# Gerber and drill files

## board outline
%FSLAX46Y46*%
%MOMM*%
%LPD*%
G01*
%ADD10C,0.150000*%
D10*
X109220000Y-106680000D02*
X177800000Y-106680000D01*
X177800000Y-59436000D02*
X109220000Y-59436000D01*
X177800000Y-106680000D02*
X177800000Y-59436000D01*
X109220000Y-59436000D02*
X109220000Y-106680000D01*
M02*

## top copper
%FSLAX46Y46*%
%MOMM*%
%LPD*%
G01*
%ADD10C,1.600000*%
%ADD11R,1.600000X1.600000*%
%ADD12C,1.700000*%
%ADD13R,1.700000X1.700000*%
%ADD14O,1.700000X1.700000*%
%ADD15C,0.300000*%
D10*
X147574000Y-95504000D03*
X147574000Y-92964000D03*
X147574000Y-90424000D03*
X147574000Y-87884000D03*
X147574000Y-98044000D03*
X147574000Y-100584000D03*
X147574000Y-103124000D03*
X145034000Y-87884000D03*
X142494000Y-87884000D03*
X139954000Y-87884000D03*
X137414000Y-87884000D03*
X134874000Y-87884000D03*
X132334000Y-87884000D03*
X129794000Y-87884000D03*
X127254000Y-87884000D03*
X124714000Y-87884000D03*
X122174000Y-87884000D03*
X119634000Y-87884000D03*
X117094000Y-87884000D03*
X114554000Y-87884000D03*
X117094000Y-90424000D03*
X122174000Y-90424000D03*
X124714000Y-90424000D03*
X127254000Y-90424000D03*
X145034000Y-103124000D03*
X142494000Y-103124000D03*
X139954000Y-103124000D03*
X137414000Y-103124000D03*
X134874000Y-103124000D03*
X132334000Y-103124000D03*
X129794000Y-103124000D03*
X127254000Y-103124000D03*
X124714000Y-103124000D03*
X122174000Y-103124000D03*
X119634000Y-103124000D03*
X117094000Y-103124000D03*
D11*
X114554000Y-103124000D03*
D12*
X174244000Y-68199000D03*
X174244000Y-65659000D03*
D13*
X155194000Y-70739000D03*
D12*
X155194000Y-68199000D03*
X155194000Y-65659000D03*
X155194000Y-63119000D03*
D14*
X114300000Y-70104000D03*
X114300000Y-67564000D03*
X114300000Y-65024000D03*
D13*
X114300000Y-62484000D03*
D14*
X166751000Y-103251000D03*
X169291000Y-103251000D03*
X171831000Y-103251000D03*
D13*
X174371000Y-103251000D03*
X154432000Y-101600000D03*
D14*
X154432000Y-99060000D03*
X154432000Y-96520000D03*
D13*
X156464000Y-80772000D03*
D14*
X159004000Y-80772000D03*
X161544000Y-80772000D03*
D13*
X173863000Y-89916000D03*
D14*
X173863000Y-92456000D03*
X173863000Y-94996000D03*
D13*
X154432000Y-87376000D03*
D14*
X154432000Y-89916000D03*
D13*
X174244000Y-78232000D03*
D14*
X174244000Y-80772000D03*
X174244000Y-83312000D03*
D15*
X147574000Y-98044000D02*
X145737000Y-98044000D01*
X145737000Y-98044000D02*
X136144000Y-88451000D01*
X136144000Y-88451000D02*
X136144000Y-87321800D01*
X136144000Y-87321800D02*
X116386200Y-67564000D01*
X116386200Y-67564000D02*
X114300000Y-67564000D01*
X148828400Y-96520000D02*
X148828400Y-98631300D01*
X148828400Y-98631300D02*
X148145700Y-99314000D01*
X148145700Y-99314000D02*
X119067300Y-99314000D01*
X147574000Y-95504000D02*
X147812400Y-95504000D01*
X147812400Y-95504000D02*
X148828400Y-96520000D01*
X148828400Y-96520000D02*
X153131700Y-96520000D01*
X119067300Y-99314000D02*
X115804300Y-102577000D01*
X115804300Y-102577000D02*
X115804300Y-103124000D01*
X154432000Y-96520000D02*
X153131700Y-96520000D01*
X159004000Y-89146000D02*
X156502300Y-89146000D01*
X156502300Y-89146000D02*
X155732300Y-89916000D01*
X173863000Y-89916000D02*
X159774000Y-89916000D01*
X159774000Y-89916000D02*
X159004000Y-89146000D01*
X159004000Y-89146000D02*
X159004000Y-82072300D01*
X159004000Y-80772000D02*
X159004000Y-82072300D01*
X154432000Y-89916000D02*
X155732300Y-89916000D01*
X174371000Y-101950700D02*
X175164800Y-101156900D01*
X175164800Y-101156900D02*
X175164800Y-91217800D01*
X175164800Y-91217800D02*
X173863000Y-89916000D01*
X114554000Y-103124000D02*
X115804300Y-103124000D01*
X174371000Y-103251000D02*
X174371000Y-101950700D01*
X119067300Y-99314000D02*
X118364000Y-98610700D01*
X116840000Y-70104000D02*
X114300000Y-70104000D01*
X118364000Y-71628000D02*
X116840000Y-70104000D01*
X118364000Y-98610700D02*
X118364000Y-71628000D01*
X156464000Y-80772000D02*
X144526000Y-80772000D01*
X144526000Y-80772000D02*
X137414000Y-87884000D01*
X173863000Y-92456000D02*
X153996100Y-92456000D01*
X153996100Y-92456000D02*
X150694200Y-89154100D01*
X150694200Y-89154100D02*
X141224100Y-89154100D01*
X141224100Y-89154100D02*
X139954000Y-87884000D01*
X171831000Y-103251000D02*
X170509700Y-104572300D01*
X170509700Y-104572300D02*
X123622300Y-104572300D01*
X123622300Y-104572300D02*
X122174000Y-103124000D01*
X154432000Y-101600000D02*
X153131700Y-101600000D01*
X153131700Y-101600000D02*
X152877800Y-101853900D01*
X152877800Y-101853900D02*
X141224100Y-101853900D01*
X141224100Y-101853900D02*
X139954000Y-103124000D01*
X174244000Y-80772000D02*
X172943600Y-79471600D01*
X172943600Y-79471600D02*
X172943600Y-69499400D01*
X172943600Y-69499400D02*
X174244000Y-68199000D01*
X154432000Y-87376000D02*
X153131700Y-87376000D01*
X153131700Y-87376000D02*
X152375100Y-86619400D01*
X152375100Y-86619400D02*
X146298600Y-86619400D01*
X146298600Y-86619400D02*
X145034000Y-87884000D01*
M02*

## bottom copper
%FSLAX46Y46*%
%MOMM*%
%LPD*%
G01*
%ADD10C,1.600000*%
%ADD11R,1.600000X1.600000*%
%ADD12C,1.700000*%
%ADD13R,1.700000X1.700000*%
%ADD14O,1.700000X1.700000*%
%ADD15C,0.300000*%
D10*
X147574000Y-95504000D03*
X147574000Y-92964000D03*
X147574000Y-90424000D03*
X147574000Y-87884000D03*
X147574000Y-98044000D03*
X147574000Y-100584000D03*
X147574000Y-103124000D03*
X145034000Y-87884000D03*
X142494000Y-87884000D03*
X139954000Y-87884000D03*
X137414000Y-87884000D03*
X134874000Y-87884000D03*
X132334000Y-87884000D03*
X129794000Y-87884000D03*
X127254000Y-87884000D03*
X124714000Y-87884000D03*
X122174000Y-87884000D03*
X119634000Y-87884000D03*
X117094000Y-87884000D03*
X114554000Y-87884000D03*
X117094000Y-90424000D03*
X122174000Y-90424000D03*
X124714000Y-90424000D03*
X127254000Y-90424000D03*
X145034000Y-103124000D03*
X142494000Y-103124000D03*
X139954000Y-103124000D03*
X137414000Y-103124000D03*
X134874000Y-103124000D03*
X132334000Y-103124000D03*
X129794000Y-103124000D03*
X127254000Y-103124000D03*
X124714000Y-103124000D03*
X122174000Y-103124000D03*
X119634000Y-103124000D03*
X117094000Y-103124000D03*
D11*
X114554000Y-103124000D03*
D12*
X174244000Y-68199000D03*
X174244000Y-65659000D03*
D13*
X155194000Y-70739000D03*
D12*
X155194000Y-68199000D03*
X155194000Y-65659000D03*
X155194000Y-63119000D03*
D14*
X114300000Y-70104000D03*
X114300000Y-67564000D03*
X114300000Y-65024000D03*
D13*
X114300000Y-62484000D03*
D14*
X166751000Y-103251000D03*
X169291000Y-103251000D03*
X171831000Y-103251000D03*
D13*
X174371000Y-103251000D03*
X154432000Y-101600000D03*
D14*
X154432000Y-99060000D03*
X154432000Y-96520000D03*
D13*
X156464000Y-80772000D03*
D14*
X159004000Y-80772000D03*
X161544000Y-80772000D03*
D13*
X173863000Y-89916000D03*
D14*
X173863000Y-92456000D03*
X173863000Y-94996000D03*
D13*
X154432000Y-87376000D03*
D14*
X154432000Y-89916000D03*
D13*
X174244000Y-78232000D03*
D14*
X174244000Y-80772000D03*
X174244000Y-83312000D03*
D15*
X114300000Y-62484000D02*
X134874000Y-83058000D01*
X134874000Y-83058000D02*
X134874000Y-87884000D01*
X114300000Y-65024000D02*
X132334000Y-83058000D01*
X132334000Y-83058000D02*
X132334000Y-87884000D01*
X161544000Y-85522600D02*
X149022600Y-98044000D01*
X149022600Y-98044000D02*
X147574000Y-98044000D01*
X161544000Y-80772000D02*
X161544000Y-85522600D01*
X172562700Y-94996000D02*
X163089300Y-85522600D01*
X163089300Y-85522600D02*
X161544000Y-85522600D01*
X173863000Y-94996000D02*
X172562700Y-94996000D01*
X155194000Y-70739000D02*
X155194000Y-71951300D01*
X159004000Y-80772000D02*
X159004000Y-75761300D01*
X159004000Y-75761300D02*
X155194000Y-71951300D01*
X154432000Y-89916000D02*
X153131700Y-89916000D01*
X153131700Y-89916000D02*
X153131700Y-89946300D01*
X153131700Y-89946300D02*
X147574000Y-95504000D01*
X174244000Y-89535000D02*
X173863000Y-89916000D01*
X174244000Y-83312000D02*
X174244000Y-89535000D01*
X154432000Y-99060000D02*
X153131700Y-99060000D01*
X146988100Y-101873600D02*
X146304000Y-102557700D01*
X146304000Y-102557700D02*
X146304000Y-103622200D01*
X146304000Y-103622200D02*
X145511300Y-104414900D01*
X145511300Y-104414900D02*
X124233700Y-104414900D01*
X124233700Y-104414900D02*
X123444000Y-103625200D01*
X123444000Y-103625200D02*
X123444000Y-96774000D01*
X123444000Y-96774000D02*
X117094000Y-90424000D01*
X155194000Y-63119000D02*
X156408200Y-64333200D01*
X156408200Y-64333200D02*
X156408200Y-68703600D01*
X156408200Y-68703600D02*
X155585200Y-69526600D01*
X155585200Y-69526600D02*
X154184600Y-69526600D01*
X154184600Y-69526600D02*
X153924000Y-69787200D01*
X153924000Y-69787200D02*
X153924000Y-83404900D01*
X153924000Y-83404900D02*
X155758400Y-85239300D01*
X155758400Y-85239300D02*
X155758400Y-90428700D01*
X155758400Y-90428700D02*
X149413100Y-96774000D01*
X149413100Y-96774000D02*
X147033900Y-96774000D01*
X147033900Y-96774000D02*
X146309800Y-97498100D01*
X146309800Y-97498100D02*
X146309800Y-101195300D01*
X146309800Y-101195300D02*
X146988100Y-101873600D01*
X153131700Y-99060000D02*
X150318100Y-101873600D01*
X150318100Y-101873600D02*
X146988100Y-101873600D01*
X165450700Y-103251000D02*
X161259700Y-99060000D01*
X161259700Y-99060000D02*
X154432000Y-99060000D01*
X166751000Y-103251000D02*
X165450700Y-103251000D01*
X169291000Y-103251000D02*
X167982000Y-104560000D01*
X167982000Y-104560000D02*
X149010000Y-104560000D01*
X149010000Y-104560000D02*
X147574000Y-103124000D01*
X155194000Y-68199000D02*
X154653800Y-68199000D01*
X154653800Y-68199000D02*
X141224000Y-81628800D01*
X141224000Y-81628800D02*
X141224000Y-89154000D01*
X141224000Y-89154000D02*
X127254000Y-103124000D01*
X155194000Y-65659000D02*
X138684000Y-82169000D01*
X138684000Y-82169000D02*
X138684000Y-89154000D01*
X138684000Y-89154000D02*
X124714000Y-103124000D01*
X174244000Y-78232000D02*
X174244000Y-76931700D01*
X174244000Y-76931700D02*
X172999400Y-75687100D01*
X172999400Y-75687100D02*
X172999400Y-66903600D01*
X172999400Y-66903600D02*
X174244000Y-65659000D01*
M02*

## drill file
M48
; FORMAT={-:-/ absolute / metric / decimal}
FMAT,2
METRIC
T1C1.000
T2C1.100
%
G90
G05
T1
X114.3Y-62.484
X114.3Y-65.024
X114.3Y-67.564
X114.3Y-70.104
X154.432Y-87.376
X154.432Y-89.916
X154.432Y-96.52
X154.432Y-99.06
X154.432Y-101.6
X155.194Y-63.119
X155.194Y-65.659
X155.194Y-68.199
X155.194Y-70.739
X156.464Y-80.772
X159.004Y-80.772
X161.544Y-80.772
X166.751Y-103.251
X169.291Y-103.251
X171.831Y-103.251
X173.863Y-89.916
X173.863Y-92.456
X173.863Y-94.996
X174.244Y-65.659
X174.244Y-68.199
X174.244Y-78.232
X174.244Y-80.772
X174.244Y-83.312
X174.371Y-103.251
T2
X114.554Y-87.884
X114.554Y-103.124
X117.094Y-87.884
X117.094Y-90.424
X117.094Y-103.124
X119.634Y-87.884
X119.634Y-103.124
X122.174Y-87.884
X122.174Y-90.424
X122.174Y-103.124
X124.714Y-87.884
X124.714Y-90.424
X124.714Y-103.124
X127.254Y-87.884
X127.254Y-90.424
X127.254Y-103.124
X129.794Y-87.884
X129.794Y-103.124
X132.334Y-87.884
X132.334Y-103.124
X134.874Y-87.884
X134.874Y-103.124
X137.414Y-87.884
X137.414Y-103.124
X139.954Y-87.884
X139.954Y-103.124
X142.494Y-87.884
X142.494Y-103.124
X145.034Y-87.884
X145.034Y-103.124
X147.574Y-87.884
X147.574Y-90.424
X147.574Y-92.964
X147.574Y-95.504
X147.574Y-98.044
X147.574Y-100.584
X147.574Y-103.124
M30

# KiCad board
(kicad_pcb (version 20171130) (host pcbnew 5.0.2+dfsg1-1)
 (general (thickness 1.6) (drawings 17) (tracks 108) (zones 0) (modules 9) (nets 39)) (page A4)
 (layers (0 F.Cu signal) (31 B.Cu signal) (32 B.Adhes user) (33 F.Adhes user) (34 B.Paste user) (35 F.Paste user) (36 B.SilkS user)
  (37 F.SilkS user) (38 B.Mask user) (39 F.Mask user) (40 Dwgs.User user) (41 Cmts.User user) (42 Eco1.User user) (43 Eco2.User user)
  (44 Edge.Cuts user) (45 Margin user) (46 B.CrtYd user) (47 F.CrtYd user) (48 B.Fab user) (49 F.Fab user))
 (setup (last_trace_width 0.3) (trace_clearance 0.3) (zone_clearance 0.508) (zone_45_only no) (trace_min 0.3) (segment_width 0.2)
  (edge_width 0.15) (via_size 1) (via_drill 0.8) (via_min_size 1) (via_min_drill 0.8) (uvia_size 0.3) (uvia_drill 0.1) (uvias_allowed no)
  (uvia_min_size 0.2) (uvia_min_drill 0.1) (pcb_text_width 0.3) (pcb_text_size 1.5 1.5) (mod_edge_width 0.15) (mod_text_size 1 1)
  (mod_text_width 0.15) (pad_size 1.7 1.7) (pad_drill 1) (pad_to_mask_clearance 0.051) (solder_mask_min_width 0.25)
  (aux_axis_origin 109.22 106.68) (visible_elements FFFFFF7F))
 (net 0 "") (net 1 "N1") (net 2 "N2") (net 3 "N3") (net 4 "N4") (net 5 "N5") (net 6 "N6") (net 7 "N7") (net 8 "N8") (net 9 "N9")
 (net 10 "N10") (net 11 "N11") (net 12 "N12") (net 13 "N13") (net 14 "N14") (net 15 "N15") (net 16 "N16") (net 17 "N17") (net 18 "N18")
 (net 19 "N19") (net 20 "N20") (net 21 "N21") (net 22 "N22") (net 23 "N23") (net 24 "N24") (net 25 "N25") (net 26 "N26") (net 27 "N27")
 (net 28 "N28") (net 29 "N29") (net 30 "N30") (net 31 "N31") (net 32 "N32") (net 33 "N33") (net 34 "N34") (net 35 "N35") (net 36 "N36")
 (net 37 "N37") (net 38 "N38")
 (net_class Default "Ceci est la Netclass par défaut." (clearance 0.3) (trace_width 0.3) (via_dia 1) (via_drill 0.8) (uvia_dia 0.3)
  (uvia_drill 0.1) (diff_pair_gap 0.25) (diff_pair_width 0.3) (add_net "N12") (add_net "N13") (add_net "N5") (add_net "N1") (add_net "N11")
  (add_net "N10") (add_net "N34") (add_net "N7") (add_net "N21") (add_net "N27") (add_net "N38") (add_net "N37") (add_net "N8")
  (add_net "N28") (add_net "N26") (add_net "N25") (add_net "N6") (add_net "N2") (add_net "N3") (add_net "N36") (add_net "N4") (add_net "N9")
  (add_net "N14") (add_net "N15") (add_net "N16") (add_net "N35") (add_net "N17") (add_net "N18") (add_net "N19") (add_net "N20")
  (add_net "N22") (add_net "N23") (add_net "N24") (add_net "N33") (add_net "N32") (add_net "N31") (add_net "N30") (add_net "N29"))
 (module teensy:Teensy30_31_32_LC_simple (layer F.Cu) (at 131.064 95.504)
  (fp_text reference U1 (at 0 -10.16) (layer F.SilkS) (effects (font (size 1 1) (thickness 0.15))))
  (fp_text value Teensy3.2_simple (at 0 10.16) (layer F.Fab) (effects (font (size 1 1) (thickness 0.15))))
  (pad 17 thru_hole circle (at 16.51 0) (size 1.6 1.6) (drill 1.1) (layers *.Cu *.Mask F.SilkS) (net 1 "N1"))
  (pad 18 thru_hole circle (at 16.51 -2.54) (size 1.6 1.6) (drill 1.1) (layers *.Cu *.Mask F.SilkS) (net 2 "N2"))
  (pad 19 thru_hole circle (at 16.51 -5.08) (size 1.6 1.6) (drill 1.1) (layers *.Cu *.Mask F.SilkS) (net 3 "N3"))
  (pad 20 thru_hole circle (at 16.51 -7.62) (size 1.6 1.6) (drill 1.1) (layers *.Cu *.Mask F.SilkS) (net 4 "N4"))
  (pad 16 thru_hole circle (at 16.51 2.54) (size 1.6 1.6) (drill 1.1) (layers *.Cu *.Mask F.SilkS) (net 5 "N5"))
  (pad 15 thru_hole circle (at 16.51 5.08) (size 1.6 1.6) (drill 1.1) (layers *.Cu *.Mask F.SilkS) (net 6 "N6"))
  (pad 14 thru_hole circle (at 16.51 7.62) (size 1.6 1.6) (drill 1.1) (layers *.Cu *.Mask F.SilkS) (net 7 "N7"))
  (pad 21 thru_hole circle (at 13.97 -7.62) (size 1.6 1.6) (drill 1.1) (layers *.Cu *.Mask F.SilkS) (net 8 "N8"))
  (pad 22 thru_hole circle (at 11.43 -7.62) (size 1.6 1.6) (drill 1.1) (layers *.Cu *.Mask F.SilkS) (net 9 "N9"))
  (pad 23 thru_hole circle (at 8.89 -7.62) (size 1.6 1.6) (drill 1.1) (layers *.Cu *.Mask F.SilkS) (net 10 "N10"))
  (pad 24 thru_hole circle (at 6.35 -7.62) (size 1.6 1.6) (drill 1.1) (layers *.Cu *.Mask F.SilkS) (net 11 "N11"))
  (pad 25 thru_hole circle (at 3.81 -7.62) (size 1.6 1.6) (drill 1.1) (layers *.Cu *.Mask F.SilkS) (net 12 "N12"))
  (pad 26 thru_hole circle (at 1.27 -7.62) (size 1.6 1.6) (drill 1.1) (layers *.Cu *.Mask F.SilkS) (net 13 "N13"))
  (pad 27 thru_hole circle (at -1.27 -7.62) (size 1.6 1.6) (drill 1.1) (layers *.Cu *.Mask F.SilkS) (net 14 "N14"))
  (pad 28 thru_hole circle (at -3.81 -7.62) (size 1.6 1.6) (drill 1.1) (layers *.Cu *.Mask F.SilkS) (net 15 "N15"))
  (pad 29 thru_hole circle (at -6.35 -7.62) (size 1.6 1.6) (drill 1.1) (layers *.Cu *.Mask F.SilkS) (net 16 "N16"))
  (pad 30 thru_hole circle (at -8.89 -7.62) (size 1.6 1.6) (drill 1.1) (layers *.Cu *.Mask F.SilkS) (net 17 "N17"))
  (pad 31 thru_hole circle (at -11.43 -7.62) (size 1.6 1.6) (drill 1.1) (layers *.Cu *.Mask F.SilkS) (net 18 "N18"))
  (pad 32 thru_hole circle (at -13.97 -7.62) (size 1.6 1.6) (drill 1.1) (layers *.Cu *.Mask F.SilkS) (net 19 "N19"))
  (pad 33 thru_hole circle (at -16.51 -7.62) (size 1.6 1.6) (drill 1.1) (layers *.Cu *.Mask F.SilkS) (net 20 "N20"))
  (pad 34 thru_hole circle (at -13.97 -5.08) (size 1.6 1.6) (drill 1.1) (layers *.Cu *.Mask F.SilkS) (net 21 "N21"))
  (pad 35 thru_hole circle (at -8.89 -5.08) (size 1.6 1.6) (drill 1.1) (layers *.Cu *.Mask F.SilkS) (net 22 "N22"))
  (pad 36 thru_hole circle (at -6.35 -5.08) (size 1.6 1.6) (drill 1.1) (layers *.Cu *.Mask F.SilkS) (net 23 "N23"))
  (pad 37 thru_hole circle (at -3.81 -5.08) (size 1.6 1.6) (drill 1.1) (layers *.Cu *.Mask F.SilkS) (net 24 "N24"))
  (pad 13 thru_hole circle (at 13.97 7.62) (size 1.6 1.6) (drill 1.1) (layers *.Cu *.Mask F.SilkS) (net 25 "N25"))
  (pad 12 thru_hole circle (at 11.43 7.62) (size 1.6 1.6) (drill 1.1) (layers *.Cu *.Mask F.SilkS) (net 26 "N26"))
  (pad 11 thru_hole circle (at 8.89 7.62) (size 1.6 1.6) (drill 1.1) (layers *.Cu *.Mask F.SilkS) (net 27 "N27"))
  (pad 10 thru_hole circle (at 6.35 7.62) (size 1.6 1.6) (drill 1.1) (layers *.Cu *.Mask F.SilkS) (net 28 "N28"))
  (pad 9 thru_hole circle (at 3.81 7.62) (size 1.6 1.6) (drill 1.1) (layers *.Cu *.Mask F.SilkS) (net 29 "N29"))
  (pad 8 thru_hole circle (at 1.27 7.62) (size 1.6 1.6) (drill 1.1) (layers *.Cu *.Mask F.SilkS) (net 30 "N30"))
  (pad 7 thru_hole circle (at -1.27 7.62) (size 1.6 1.6) (drill 1.1) (layers *.Cu *.Mask F.SilkS) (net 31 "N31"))
  (pad 6 thru_hole circle (at -3.81 7.62) (size 1.6 1.6) (drill 1.1) (layers *.Cu *.Mask F.SilkS) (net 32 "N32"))
  (pad 5 thru_hole circle (at -6.35 7.62) (size 1.6 1.6) (drill 1.1) (layers *.Cu *.Mask F.SilkS) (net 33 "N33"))
  (pad 4 thru_hole circle (at -8.89 7.62) (size 1.6 1.6) (drill 1.1) (layers *.Cu *.Mask F.SilkS) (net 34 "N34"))
  (pad 3 thru_hole circle (at -11.43 7.62) (size 1.6 1.6) (drill 1.1) (layers *.Cu *.Mask F.SilkS) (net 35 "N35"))
  (pad 2 thru_hole circle (at -13.97 7.62) (size 1.6 1.6) (drill 1.1) (layers *.Cu *.Mask F.SilkS) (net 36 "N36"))
  (pad 1 thru_hole rect (at -16.51 7.62) (size 1.6 1.6) (drill 1.1) (layers *.Cu *.Mask F.SilkS) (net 1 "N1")))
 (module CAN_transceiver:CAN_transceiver (layer F.Cu) (at 153.924 72.644)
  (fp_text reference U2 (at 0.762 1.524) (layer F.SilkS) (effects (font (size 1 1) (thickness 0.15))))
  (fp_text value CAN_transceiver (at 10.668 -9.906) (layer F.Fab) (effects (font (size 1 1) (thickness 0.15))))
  (pad 5 thru_hole circle (at 20.32 -4.445) (size 1.7 1.7) (drill 1) (layers *.Cu *.Mask) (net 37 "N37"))
  (pad 6 thru_hole circle (at 20.32 -6.985) (size 1.7 1.7) (drill 1) (layers *.Cu *.Mask) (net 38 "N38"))
  (pad 1 thru_hole rect (at 1.27 -1.905) (size 1.7 1.7) (drill 1) (layers *.Cu *.Mask) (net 1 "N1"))
  (pad 2 thru_hole circle (at 1.27 -4.445) (size 1.7 1.7) (drill 1) (layers *.Cu *.Mask) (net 32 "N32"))
  (pad 3 thru_hole circle (at 1.27 -6.985) (size 1.7 1.7) (drill 1) (layers *.Cu *.Mask) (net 33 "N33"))
  (pad 4 thru_hole circle (at 1.27 -9.525) (size 1.7 1.7) (drill 1) (layers *.Cu *.Mask) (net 21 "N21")))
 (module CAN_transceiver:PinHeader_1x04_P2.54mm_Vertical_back (layer F.Cu) (at 114.3 62.484)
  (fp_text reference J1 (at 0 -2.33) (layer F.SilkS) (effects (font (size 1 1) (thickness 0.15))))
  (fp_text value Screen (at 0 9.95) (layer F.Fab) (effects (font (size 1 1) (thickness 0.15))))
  (pad 4 thru_hole oval (at 0 7.62) (size 1.7 1.7) (drill 1) (layers *.Cu *.Mask) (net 1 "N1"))
  (pad 3 thru_hole oval (at 0 5.08) (size 1.7 1.7) (drill 1) (layers *.Cu *.Mask) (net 5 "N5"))
  (pad 2 thru_hole oval (at 0 2.54) (size 1.7 1.7) (drill 1) (layers *.Cu *.Mask) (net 13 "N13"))
  (pad 1 thru_hole rect (at 0 0) (size 1.7 1.7) (drill 1) (layers *.Cu *.Mask) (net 12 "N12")))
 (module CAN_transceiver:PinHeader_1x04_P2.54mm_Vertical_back (layer F.Cu) (at 174.371 103.251 270)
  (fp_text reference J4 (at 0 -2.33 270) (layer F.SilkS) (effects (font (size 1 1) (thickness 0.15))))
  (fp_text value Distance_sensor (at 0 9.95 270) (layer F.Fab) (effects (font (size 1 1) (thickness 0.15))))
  (pad 4 thru_hole oval (at 0 7.62 270) (size 1.7 1.7) (drill 1) (layers *.Cu *.Mask) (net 21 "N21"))
  (pad 3 thru_hole oval (at 0 5.08 270) (size 1.7 1.7) (drill 1) (layers *.Cu *.Mask) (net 7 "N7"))
  (pad 2 thru_hole oval (at 0 2.54 270) (size 1.7 1.7) (drill 1) (layers *.Cu *.Mask) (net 34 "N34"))
  (pad 1 thru_hole rect (at 0 0 270) (size 1.7 1.7) (drill 1) (layers *.Cu *.Mask) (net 1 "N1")))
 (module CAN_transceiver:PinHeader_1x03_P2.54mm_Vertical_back (layer F.Cu) (at 154.432 101.6 180)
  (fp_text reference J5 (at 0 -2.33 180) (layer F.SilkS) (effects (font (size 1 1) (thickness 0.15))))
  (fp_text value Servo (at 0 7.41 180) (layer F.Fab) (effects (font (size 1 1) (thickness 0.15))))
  (pad 1 thru_hole rect (at 0 0 180) (size 1.7 1.7) (drill 1) (layers *.Cu *.Mask) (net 27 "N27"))
  (pad 2 thru_hole oval (at 0 2.54 180) (size 1.7 1.7) (drill 1) (layers *.Cu *.Mask) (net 21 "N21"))
  (pad 3 thru_hole oval (at 0 5.08 180) (size 1.7 1.7) (drill 1) (layers *.Cu *.Mask) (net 1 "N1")))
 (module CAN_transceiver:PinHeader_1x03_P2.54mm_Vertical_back (layer F.Cu) (at 156.464 80.772 90)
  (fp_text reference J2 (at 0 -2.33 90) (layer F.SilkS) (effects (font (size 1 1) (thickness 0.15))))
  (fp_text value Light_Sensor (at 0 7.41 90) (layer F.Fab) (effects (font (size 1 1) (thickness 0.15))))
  (pad 1 thru_hole rect (at 0 0 90) (size 1.7 1.7) (drill 1) (layers *.Cu *.Mask) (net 11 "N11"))
  (pad 2 thru_hole oval (at 0 2.54 90) (size 1.7 1.7) (drill 1) (layers *.Cu *.Mask) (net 1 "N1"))
  (pad 3 thru_hole oval (at 0 5.08 90) (size 1.7 1.7) (drill 1) (layers *.Cu *.Mask) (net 5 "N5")))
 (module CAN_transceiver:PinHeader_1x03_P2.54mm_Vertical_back (layer F.Cu) (at 173.863 89.916)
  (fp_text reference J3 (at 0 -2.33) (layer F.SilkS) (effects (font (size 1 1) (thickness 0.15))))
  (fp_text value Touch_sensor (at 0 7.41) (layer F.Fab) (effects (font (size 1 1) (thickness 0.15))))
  (pad 1 thru_hole rect (at 0 0) (size 1.7 1.7) (drill 1) (layers *.Cu *.Mask) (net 1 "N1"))
  (pad 2 thru_hole oval (at 0 2.54) (size 1.7 1.7) (drill 1) (layers *.Cu *.Mask) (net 10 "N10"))
  (pad 3 thru_hole oval (at 0 5.08) (size 1.7 1.7) (drill 1) (layers *.Cu *.Mask) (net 5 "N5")))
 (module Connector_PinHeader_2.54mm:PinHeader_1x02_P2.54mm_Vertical (layer F.Cu) (at 154.432 87.376)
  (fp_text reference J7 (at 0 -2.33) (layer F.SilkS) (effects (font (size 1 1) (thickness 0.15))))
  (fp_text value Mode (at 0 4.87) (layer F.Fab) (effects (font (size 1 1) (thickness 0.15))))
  (pad 1 thru_hole rect (at 0 0) (size 1.7 1.7) (drill 1) (layers *.Cu *.Mask) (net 8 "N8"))
  (pad 2 thru_hole oval (at 0 2.54) (size 1.7 1.7) (drill 1) (layers *.Cu *.Mask) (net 1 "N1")))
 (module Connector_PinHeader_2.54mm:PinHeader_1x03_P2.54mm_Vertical (layer F.Cu) (at 174.244 78.232)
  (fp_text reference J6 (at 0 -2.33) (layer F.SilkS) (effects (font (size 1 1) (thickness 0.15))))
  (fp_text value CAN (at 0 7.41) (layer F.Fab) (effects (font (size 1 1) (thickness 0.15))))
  (pad 1 thru_hole rect (at 0 0) (size 1.7 1.7) (drill 1) (layers *.Cu *.Mask) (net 38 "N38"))
  (pad 2 thru_hole oval (at 0 2.54) (size 1.7 1.7) (drill 1) (layers *.Cu *.Mask) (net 37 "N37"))
  (pad 3 thru_hole oval (at 0 5.08) (size 1.7 1.7) (drill 1) (layers *.Cu *.Mask) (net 1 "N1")))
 (gr_line (start 109.22 106.68) (end 177.8 106.68) (layer Edge.Cuts) (width 0.15))
 (gr_line (start 177.8 59.436) (end 109.22 59.436) (layer Edge.Cuts) (width 0.15))
 (gr_line (start 177.8 106.68) (end 177.8 59.436) (layer Edge.Cuts) (width 0.15))
 (gr_line (start 109.22 59.436) (end 109.22 106.68) (layer Edge.Cuts) (width 0.15))
 (segment (start 114.3 62.484) (end 134.874 83.058) (width 0.3) (layer B.Cu) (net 12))
 (segment (start 134.874 83.058) (end 134.874 87.884) (width 0.3) (layer B.Cu) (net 12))
 (segment (start 114.3 65.024) (end 132.334 83.058) (width 0.3) (layer B.Cu) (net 13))
 (segment (start 132.334 83.058) (end 132.334 87.884) (width 0.3) (layer B.Cu) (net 13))
 (segment (start 161.544 85.5226) (end 149.0226 98.044) (width 0.3) (layer B.Cu) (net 5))
 (segment (start 149.0226 98.044) (end 147.574 98.044) (width 0.3) (layer B.Cu) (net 5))
 (segment (start 161.544 80.772) (end 161.544 85.5226) (width 0.3) (layer B.Cu) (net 5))
 (segment (start 172.5627 94.996) (end 163.0893 85.5226) (width 0.3) (layer B.Cu) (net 5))
 (segment (start 163.0893 85.5226) (end 161.544 85.5226) (width 0.3) (layer B.Cu) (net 5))
 (segment (start 173.863 94.996) (end 172.5627 94.996) (width 0.3) (layer B.Cu) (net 5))
 (segment (start 147.574 98.044) (end 145.737 98.044) (width 0.3) (layer F.Cu) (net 5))
 (segment (start 145.737 98.044) (end 136.144 88.451) (width 0.3) (layer F.Cu) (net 5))
 (segment (start 136.144 88.451) (end 136.144 87.3218) (width 0.3) (layer F.Cu) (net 5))
 (segment (start 136.144 87.3218) (end 116.3862 67.564) (width 0.3) (layer F.Cu) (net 5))
 (segment (start 116.3862 67.564) (end 114.3 67.564) (width 0.3) (layer F.Cu) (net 5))
 (segment (start 155.194 70.739) (end 155.194 71.9513) (width 0.3) (layer B.Cu) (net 1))
 (segment (start 159.004 80.772) (end 159.004 75.7613) (width 0.3) (layer B.Cu) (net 1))
 (segment (start 159.004 75.7613) (end 155.194 71.9513) (width 0.3) (layer B.Cu) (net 1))
 (segment (start 154.432 89.916) (end 153.1317 89.916) (width 0.3) (layer B.Cu) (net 1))
 (segment (start 153.1317 89.916) (end 153.1317 89.9463) (width 0.3) (layer B.Cu) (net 1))
 (segment (start 153.1317 89.9463) (end 147.574 95.504) (width 0.3) (layer B.Cu) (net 1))
 (segment (start 148.8284 96.52) (end 148.8284 98.6313) (width 0.3) (layer F.Cu) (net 1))
 (segment (start 148.8284 98.6313) (end 148.1457 99.314) (width 0.3) (layer F.Cu) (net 1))
 (segment (start 148.1457 99.314) (end 119.0673 99.314) (width 0.3) (layer F.Cu) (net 1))
 (segment (start 147.574 95.504) (end 147.8124 95.504) (width 0.3) (layer F.Cu) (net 1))
 (segment (start 147.8124 95.504) (end 148.8284 96.52) (width 0.3) (layer F.Cu) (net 1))
 (segment (start 148.8284 96.52) (end 153.1317 96.52) (width 0.3) (layer F.Cu) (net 1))
 (segment (start 119.0673 99.314) (end 115.8043 102.577) (width 0.3) (layer F.Cu) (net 1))
 (segment (start 115.8043 102.577) (end 115.8043 103.124) (width 0.3) (layer F.Cu) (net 1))
 (segment (start 154.432 96.52) (end 153.1317 96.52) (width 0.3) (layer F.Cu) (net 1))
 (segment (start 159.004 89.146) (end 156.5023 89.146) (width 0.3) (layer F.Cu) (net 1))
 (segment (start 156.5023 89.146) (end 155.7323 89.916) (width 0.3) (layer F.Cu) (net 1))
 (segment (start 173.863 89.916) (end 159.774 89.916) (width 0.3) (layer F.Cu) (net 1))
 (segment (start 159.774 89.916) (end 159.004 89.146) (width 0.3) (layer F.Cu) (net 1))
 (segment (start 159.004 89.146) (end 159.004 82.0723) (width 0.3) (layer F.Cu) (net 1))
 (segment (start 159.004 80.772) (end 159.004 82.0723) (width 0.3) (layer F.Cu) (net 1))
 (segment (start 154.432 89.916) (end 155.7323 89.916) (width 0.3) (layer F.Cu) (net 1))
 (segment (start 174.371 101.9507) (end 175.1648 101.1569) (width 0.3) (layer F.Cu) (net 1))
 (segment (start 175.1648 101.1569) (end 175.1648 91.2178) (width 0.3) (layer F.Cu) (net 1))
 (segment (start 175.1648 91.2178) (end 173.863 89.916) (width 0.3) (layer F.Cu) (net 1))
 (segment (start 114.554 103.124) (end 115.8043 103.124) (width 0.3) (layer F.Cu) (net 1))
 (segment (start 174.371 103.251) (end 174.371 101.9507) (width 0.3) (layer F.Cu) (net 1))
 (segment (start 119.0673 99.314) (end 118.364 98.6107) (width 0.3) (layer F.Cu) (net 1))
 (segment (start 116.84 70.104) (end 114.3 70.104) (width 0.3) (layer F.Cu) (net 1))
 (segment (start 118.364 71.628) (end 116.84 70.104) (width 0.3) (layer F.Cu) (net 1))
 (segment (start 118.364 98.6107) (end 118.364 71.628) (width 0.3) (layer F.Cu) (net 1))
 (segment (start 174.244 89.535) (end 173.863 89.916) (width 0.3) (layer B.Cu) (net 1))
 (segment (start 174.244 83.312) (end 174.244 89.535) (width 0.3) (layer B.Cu) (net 1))
 (segment (start 156.464 80.772) (end 144.526 80.772) (width 0.3) (layer F.Cu) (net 11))
 (segment (start 144.526 80.772) (end 137.414 87.884) (width 0.3) (layer F.Cu) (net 11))
 (segment (start 173.863 92.456) (end 153.9961 92.456) (width 0.3) (layer F.Cu) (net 10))
 (segment (start 153.9961 92.456) (end 150.6942 89.1541) (width 0.3) (layer F.Cu) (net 10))
 (segment (start 150.6942 89.1541) (end 141.2241 89.1541) (width 0.3) (layer F.Cu) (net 10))
 (segment (start 141.2241 89.1541) (end 139.954 87.884) (width 0.3) (layer F.Cu) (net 10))
 (segment (start 154.432 99.06) (end 153.1317 99.06) (width 0.3) (layer B.Cu) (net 21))
 (segment (start 146.9881 101.8736) (end 146.304 102.5577) (width 0.3) (layer B.Cu) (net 21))
 (segment (start 146.304 102.5577) (end 146.304 103.6222) (width 0.3) (layer B.Cu) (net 21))
 (segment (start 146.304 103.6222) (end 145.5113 104.4149) (width 0.3) (layer B.Cu) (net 21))
 (segment (start 145.5113 104.4149) (end 124.2337 104.4149) (width 0.3) (layer B.Cu) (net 21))
 (segment (start 124.2337 104.4149) (end 123.444 103.6252) (width 0.3) (layer B.Cu) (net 21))
 (segment (start 123.444 103.6252) (end 123.444 96.774) (width 0.3) (layer B.Cu) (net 21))
 (segment (start 123.444 96.774) (end 117.094 90.424) (width 0.3) (layer B.Cu) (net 21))
 (segment (start 155.194 63.119) (end 156.4082 64.3332) (width 0.3) (layer B.Cu) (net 21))
 (segment (start 156.4082 64.3332) (end 156.4082 68.7036) (width 0.3) (layer B.Cu) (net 21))
 (segment (start 156.4082 68.7036) (end 155.5852 69.5266) (width 0.3) (layer B.Cu) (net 21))
 (segment (start 155.5852 69.5266) (end 154.1846 69.5266) (width 0.3) (layer B.Cu) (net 21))
 (segment (start 154.1846 69.5266) (end 153.924 69.7872) (width 0.3) (layer B.Cu) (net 21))
 (segment (start 153.924 69.7872) (end 153.924 83.4049) (width 0.3) (layer B.Cu) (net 21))
 (segment (start 153.924 83.4049) (end 155.7584 85.2393) (width 0.3) (layer B.Cu) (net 21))
 (segment (start 155.7584 85.2393) (end 155.7584 90.4287) (width 0.3) (layer B.Cu) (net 21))
 (segment (start 155.7584 90.4287) (end 149.4131 96.774) (width 0.3) (layer B.Cu) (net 21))
 (segment (start 149.4131 96.774) (end 147.0339 96.774) (width 0.3) (layer B.Cu) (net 21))
 (segment (start 147.0339 96.774) (end 146.3098 97.4981) (width 0.3) (layer B.Cu) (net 21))
 (segment (start 146.3098 97.4981) (end 146.3098 101.1953) (width 0.3) (layer B.Cu) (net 21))
 (segment (start 146.3098 101.1953) (end 146.9881 101.8736) (width 0.3) (layer B.Cu) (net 21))
 (segment (start 153.1317 99.06) (end 150.3181 101.8736) (width 0.3) (layer B.Cu) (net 21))
 (segment (start 150.3181 101.8736) (end 146.9881 101.8736) (width 0.3) (layer B.Cu) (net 21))
 (segment (start 165.4507 103.251) (end 161.2597 99.06) (width 0.3) (layer B.Cu) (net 21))
 (segment (start 161.2597 99.06) (end 154.432 99.06) (width 0.3) (layer B.Cu) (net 21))
 (segment (start 166.751 103.251) (end 165.4507 103.251) (width 0.3) (layer B.Cu) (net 21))
 (segment (start 169.291 103.251) (end 167.982 104.56) (width 0.3) (layer B.Cu) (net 7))
 (segment (start 167.982 104.56) (end 149.01 104.56) (width 0.3) (layer B.Cu) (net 7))
 (segment (start 149.01 104.56) (end 147.574 103.124) (width 0.3) (layer B.Cu) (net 7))
 (segment (start 171.831 103.251) (end 170.5097 104.5723) (width 0.3) (layer F.Cu) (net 34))
 (segment (start 170.5097 104.5723) (end 123.6223 104.5723) (width 0.3) (layer F.Cu) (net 34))
 (segment (start 123.6223 104.5723) (end 122.174 103.124) (width 0.3) (layer F.Cu) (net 34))
 (segment (start 154.432 101.6) (end 153.1317 101.6) (width 0.3) (layer F.Cu) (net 27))
 (segment (start 153.1317 101.6) (end 152.8778 101.8539) (width 0.3) (layer F.Cu) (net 27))
 (segment (start 152.8778 101.8539) (end 141.2241 101.8539) (width 0.3) (layer F.Cu) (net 27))
 (segment (start 141.2241 101.8539) (end 139.954 103.124) (width 0.3) (layer F.Cu) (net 27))
 (segment (start 155.194 68.199) (end 154.6538 68.199) (width 0.3) (layer B.Cu) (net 32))
 (segment (start 154.6538 68.199) (end 141.224 81.6288) (width 0.3) (layer B.Cu) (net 32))
 (segment (start 141.224 81.6288) (end 141.224 89.154) (width 0.3) (layer B.Cu) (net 32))
 (segment (start 141.224 89.154) (end 127.254 103.124) (width 0.3) (layer B.Cu) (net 32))
 (segment (start 155.194 65.659) (end 138.684 82.169) (width 0.3) (layer B.Cu) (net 33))
 (segment (start 138.684 82.169) (end 138.684 89.154) (width 0.3) (layer B.Cu) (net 33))
 (segment (start 138.684 89.154) (end 124.714 103.124) (width 0.3) (layer B.Cu) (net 33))
 (segment (start 174.244 80.772) (end 172.9436 79.4716) (width 0.3) (layer F.Cu) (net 37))
 (segment (start 172.9436 79.4716) (end 172.9436 69.4994) (width 0.3) (layer F.Cu) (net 37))
 (segment (start 172.9436 69.4994) (end 174.244 68.199) (width 0.3) (layer F.Cu) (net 37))
 (segment (start 174.244 78.232) (end 174.244 76.9317) (width 0.3) (layer B.Cu) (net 38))
 (segment (start 174.244 76.9317) (end 172.9994 75.6871) (width 0.3) (layer B.Cu) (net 38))
 (segment (start 172.9994 75.6871) (end 172.9994 66.9036) (width 0.3) (layer B.Cu) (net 38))
 (segment (start 172.9994 66.9036) (end 174.244 65.659) (width 0.3) (layer B.Cu) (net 38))
 (segment (start 154.432 87.376) (end 153.1317 87.376) (width 0.3) (layer F.Cu) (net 8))
 (segment (start 153.1317 87.376) (end 152.3751 86.6194) (width 0.3) (layer F.Cu) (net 8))
 (segment (start 152.3751 86.6194) (end 146.2986 86.6194) (width 0.3) (layer F.Cu) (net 8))
 (segment (start 146.2986 86.6194) (end 145.034 87.884) (width 0.3) (layer F.Cu) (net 8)))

